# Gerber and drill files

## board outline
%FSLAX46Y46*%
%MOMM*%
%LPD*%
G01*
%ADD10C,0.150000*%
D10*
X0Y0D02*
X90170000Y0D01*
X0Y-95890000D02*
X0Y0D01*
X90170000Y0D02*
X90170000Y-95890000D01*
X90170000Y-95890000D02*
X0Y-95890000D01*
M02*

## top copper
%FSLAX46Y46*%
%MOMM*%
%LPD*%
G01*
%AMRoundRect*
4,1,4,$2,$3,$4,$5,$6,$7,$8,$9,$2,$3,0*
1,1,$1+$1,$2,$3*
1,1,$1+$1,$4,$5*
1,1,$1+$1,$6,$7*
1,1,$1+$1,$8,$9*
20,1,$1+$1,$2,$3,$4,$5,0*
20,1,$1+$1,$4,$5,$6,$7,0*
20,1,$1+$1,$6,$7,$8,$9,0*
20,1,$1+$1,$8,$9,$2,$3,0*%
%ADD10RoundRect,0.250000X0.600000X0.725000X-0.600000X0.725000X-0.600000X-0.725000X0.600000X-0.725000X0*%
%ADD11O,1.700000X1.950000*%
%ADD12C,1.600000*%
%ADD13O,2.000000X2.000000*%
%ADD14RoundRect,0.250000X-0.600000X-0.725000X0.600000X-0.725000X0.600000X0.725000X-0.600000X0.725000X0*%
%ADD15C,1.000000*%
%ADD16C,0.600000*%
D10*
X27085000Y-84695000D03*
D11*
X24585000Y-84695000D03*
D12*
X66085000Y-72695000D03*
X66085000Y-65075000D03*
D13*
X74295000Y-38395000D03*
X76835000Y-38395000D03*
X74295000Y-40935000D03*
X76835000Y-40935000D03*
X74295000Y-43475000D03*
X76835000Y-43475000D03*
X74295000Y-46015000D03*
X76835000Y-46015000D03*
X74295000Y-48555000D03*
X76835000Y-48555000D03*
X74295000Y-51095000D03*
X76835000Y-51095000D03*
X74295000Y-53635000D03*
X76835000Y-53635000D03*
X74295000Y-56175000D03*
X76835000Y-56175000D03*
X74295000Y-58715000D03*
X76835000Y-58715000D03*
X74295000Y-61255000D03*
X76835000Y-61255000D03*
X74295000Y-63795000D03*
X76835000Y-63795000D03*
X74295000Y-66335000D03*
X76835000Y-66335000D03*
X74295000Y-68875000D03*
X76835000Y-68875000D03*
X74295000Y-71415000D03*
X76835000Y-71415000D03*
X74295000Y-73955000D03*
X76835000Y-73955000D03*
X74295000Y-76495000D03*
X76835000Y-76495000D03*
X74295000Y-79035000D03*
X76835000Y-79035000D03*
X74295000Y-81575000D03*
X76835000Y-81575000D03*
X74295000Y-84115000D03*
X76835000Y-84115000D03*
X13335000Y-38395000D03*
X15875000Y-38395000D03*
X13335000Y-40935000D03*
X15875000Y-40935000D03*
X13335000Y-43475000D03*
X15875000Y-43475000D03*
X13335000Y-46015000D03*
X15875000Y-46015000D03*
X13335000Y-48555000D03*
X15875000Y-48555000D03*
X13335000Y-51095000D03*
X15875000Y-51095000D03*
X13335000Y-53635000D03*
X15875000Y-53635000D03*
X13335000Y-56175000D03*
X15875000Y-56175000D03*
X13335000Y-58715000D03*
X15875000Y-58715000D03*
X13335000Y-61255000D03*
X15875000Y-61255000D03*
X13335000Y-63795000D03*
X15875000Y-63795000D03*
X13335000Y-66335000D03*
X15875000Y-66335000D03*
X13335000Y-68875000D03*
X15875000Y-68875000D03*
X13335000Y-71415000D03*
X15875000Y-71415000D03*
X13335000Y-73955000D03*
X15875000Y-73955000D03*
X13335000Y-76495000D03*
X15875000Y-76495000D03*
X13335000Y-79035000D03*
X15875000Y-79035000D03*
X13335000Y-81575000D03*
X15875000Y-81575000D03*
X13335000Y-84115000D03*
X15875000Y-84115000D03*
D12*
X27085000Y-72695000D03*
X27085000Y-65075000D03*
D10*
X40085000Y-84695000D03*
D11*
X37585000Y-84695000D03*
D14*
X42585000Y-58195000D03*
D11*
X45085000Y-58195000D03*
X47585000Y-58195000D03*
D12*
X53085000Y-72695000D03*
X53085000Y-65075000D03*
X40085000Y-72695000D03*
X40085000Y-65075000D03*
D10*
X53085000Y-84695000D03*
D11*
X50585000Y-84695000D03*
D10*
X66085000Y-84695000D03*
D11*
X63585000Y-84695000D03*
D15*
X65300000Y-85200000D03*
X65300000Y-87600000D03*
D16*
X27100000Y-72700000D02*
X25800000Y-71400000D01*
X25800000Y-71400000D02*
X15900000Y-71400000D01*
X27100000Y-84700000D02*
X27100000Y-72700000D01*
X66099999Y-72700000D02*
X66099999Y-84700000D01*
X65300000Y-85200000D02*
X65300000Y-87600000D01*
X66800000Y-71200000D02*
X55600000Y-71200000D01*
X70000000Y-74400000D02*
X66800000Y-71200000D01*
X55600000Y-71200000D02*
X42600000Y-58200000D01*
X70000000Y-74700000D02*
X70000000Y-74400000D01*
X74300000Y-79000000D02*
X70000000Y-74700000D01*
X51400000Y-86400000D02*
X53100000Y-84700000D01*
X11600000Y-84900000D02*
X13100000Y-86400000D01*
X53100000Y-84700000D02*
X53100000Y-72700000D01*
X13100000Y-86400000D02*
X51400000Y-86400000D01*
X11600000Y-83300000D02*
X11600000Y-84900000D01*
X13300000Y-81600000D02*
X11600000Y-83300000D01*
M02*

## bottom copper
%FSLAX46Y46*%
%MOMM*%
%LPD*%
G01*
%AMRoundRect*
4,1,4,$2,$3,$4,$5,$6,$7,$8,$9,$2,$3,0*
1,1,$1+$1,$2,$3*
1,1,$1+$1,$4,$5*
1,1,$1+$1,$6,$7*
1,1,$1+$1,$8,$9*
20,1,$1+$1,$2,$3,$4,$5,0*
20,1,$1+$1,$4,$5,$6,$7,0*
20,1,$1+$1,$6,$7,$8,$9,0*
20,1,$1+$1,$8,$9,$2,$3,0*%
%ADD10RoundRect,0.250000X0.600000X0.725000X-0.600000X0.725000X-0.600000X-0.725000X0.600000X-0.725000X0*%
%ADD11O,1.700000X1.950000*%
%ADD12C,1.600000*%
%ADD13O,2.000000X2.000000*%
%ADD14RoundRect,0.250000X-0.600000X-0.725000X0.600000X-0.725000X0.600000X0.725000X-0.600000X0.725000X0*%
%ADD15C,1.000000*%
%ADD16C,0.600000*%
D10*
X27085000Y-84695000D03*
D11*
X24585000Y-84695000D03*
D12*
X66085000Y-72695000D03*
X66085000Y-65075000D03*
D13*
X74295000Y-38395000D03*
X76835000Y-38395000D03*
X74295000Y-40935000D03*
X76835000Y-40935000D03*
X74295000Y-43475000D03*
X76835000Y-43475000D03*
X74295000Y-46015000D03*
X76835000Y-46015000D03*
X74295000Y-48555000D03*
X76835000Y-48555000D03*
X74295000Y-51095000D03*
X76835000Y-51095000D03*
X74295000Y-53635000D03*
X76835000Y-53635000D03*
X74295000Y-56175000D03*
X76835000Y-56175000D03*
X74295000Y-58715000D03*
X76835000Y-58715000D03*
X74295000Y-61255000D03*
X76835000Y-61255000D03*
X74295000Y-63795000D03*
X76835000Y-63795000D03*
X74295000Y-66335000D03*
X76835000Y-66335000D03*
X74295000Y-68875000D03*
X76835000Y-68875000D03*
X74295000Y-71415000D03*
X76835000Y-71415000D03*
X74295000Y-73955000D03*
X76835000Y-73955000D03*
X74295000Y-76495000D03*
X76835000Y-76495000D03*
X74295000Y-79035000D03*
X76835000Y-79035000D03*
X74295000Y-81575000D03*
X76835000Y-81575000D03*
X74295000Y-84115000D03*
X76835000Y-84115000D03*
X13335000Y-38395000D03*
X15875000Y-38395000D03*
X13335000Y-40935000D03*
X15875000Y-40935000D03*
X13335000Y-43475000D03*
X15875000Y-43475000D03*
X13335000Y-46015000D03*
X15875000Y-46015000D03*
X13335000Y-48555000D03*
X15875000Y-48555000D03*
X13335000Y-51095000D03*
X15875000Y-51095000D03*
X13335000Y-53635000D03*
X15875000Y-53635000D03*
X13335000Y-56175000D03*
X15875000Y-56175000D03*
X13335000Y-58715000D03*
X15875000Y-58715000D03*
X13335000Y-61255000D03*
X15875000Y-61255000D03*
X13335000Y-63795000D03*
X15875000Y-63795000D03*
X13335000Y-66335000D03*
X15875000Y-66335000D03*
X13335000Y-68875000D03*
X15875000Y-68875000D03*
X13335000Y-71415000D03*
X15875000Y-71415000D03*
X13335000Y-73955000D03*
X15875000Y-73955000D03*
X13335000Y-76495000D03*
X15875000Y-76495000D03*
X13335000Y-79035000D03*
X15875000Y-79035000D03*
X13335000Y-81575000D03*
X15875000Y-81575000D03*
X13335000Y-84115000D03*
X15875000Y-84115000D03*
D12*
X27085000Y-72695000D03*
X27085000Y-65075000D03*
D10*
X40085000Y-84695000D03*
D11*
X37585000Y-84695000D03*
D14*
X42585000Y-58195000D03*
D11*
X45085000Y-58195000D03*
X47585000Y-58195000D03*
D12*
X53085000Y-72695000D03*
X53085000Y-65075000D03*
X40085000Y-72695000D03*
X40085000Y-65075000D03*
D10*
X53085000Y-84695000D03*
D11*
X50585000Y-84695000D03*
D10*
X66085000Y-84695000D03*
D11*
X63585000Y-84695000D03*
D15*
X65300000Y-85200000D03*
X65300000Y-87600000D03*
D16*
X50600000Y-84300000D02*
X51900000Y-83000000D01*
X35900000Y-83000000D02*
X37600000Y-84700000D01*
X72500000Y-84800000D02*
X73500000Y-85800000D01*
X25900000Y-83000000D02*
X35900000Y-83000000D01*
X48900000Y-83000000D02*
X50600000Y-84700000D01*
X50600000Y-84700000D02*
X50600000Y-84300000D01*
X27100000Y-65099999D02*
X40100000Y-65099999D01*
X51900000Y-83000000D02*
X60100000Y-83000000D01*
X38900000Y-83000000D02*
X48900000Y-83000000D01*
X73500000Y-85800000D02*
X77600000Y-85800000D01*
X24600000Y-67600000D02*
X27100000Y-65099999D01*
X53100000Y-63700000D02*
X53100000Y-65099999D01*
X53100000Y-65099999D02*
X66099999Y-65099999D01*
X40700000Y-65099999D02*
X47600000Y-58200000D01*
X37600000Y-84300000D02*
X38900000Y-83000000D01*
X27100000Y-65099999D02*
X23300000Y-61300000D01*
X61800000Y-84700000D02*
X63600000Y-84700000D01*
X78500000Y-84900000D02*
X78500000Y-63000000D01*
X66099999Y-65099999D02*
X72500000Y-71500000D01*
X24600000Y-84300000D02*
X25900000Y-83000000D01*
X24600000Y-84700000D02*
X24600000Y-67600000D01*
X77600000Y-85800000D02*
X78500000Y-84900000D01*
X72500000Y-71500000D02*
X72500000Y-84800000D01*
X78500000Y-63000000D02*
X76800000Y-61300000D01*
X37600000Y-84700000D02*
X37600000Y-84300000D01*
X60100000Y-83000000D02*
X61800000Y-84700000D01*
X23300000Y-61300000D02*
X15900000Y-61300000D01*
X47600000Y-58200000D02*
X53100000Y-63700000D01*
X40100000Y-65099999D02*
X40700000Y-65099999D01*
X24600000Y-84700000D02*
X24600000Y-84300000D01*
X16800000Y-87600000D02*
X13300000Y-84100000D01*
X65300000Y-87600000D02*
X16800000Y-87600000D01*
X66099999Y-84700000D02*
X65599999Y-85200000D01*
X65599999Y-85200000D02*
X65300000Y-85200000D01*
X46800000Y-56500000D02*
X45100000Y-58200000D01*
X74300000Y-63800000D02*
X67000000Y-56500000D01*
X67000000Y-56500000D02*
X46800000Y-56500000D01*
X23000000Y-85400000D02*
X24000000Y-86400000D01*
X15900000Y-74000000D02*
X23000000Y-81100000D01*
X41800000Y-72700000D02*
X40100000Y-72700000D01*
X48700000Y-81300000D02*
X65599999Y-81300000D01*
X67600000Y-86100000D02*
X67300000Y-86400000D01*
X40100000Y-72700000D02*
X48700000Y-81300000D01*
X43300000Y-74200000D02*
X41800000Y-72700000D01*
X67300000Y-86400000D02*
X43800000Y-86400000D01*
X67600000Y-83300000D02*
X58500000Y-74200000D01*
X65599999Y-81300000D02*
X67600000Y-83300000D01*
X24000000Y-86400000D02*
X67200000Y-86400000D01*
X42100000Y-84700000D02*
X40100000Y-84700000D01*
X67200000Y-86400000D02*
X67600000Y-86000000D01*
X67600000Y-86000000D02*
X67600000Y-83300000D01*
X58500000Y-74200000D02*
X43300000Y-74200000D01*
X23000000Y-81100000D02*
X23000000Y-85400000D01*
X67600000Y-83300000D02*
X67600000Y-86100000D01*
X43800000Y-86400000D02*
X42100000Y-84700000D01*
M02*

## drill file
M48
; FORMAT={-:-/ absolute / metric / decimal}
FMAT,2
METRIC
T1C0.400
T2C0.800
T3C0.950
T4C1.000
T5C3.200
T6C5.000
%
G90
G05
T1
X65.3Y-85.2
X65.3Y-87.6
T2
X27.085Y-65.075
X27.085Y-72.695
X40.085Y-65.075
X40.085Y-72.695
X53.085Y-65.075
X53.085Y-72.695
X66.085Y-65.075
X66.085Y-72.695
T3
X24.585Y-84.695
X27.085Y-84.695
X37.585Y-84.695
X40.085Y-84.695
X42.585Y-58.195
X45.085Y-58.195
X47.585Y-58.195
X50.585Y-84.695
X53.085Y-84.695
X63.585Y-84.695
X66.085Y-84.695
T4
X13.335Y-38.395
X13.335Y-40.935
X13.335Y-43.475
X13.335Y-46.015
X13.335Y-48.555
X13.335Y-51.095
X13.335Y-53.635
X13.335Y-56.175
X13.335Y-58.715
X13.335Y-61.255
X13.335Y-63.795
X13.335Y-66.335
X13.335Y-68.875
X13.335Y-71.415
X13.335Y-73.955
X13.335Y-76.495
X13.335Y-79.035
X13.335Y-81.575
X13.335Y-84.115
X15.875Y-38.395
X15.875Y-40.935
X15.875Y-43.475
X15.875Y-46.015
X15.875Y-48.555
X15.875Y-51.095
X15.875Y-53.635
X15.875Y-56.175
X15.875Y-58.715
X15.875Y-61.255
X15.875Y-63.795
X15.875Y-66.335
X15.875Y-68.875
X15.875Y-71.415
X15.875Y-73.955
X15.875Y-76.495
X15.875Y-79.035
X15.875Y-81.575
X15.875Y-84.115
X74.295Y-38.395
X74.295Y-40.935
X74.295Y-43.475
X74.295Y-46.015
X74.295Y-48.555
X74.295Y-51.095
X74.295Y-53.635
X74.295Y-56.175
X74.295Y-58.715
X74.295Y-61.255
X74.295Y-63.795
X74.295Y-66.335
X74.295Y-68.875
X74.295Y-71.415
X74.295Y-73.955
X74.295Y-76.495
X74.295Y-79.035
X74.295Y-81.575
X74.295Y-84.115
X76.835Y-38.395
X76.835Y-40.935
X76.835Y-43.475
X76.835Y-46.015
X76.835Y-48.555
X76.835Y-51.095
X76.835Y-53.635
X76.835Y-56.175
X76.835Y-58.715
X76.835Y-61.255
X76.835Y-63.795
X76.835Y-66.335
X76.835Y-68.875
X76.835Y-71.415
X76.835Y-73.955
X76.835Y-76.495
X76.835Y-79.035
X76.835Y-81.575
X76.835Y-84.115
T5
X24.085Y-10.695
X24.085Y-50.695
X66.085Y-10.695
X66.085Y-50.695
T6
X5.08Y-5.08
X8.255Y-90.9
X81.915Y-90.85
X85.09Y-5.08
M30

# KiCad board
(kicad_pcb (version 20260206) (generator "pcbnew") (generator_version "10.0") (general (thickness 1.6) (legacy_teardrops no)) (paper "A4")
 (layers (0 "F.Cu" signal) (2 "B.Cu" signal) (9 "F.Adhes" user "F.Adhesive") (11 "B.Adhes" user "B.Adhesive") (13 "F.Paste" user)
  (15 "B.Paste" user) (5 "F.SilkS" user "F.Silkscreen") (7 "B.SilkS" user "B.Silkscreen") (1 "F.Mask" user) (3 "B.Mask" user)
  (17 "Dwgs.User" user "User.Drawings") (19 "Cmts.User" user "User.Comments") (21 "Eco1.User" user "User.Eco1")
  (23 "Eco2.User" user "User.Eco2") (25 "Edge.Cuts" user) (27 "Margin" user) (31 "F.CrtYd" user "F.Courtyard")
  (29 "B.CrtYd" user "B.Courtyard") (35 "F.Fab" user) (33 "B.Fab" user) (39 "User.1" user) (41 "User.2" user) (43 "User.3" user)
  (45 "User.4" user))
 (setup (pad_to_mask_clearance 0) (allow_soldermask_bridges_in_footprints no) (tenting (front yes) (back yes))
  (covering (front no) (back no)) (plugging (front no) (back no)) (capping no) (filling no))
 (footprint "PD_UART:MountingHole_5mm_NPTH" (layer "F.Cu") (at 8.255 90.9)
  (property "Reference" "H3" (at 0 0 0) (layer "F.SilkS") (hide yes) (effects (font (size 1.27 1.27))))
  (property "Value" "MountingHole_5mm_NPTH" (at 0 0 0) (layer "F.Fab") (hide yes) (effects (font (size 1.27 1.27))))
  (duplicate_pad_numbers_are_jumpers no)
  (pad "" np_thru_hole circle (at 0 0) (size 5 5) (drill 5) (layers "*.Cu")))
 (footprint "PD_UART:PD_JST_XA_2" (layer "F.Cu") (at 27.085 84.695 180)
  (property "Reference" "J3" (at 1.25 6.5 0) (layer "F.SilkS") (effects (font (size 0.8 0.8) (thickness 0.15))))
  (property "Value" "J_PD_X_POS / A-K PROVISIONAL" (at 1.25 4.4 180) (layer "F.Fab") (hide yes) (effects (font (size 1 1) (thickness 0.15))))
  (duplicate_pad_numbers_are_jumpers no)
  (pad "1" thru_hole roundrect (at 0 0 180) (size 1.7 1.95) (drill 0.95) (layers "*.Cu") (remove_unused_layers no)
   (roundrect_rratio 0.147059) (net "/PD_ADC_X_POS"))
  (pad "2" thru_hole oval (at 2.5 0 180) (size 1.7 1.95) (drill 0.95) (layers "*.Cu") (remove_unused_layers no) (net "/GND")))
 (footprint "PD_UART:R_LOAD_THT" (layer "F.Cu") (at 66.085 72.695 90)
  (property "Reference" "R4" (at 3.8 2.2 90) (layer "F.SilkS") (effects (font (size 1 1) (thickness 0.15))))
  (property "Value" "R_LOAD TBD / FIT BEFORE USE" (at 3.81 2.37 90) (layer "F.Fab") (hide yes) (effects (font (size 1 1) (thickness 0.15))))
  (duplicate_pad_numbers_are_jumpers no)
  (pad "1" thru_hole circle (at 0 0 90) (size 1.6 1.6) (drill 0.8) (layers "*.Cu") (remove_unused_layers no) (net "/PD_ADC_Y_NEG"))
  (pad "2" thru_hole circle (at 7.62 0 90) (size 1.6 1.6) (drill 0.8) (layers "*.Cu") (remove_unused_layers no) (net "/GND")))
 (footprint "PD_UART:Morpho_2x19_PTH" (layer "F.Cu") (at 74.295 38.395)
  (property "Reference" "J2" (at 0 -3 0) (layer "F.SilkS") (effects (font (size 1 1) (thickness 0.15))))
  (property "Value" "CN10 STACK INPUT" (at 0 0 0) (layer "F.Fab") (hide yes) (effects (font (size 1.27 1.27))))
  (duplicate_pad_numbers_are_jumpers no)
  (pad "1" thru_hole oval (at 0 0) (size 2 2) (drill 1) (layers "*.Cu") (remove_unused_layers no) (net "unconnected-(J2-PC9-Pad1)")
   (thermal_bridge_angle 45))
  (pad "2" thru_hole oval (at 2.54 0) (size 2 2) (drill 1) (layers "*.Cu") (remove_unused_layers no) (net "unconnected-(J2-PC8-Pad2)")
   (thermal_bridge_angle 45))
  (pad "3" thru_hole oval (at 0 2.54) (size 2 2) (drill 1) (layers "*.Cu") (remove_unused_layers no) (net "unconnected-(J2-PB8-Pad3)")
   (thermal_bridge_angle 45))
  (pad "4" thru_hole oval (at 2.54 2.54) (size 2 2) (drill 1) (layers "*.Cu") (remove_unused_layers no) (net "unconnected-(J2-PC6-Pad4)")
   (thermal_bridge_angle 45))
  (pad "5" thru_hole oval (at 0 5.08) (size 2 2) (drill 1) (layers "*.Cu") (remove_unused_layers no) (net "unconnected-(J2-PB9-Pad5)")
   (thermal_bridge_angle 45))
  (pad "6" thru_hole oval (at 2.54 5.08) (size 2 2) (drill 1) (layers "*.Cu") (remove_unused_layers no) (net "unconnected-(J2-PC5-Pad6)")
   (thermal_bridge_angle 45))
  (pad "7" thru_hole oval (at 0 7.62) (size 2 2) (drill 1) (layers "*.Cu") (remove_unused_layers no) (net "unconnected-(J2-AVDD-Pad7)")
   (thermal_bridge_angle 45))
  (pad "8" thru_hole oval (at 2.54 7.62) (size 2 2) (drill 1) (layers "*.Cu") (remove_unused_layers no) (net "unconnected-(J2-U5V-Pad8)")
   (thermal_bridge_angle 45))
  (pad "9" thru_hole oval (at 0 10.16) (size 2 2) (drill 1) (layers "*.Cu") (remove_unused_layers no) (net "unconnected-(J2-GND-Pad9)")
   (thermal_bridge_angle 45))
  (pad "10" thru_hole oval (at 2.54 10.16) (size 2 2) (drill 1) (layers "*.Cu") (remove_unused_layers no) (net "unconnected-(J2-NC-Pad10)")
   (thermal_bridge_angle 45))
  (pad "11" thru_hole oval (at 0 12.7) (size 2 2) (drill 1) (layers "*.Cu") (remove_unused_layers no) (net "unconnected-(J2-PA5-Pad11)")
   (thermal_bridge_angle 45))
  (pad "12" thru_hole oval (at 2.54 12.7) (size 2 2) (drill 1) (layers "*.Cu") (remove_unused_layers no) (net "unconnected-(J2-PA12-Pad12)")
   (thermal_bridge_angle 45))
  (pad "13" thru_hole oval (at 0 15.24) (size 2 2) (drill 1) (layers "*.Cu") (remove_unused_layers no) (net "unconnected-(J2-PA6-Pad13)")
   (thermal_bridge_angle 45))
  (pad "14" thru_hole oval (at 2.54 15.24) (size 2 2) (drill 1) (layers "*.Cu") (remove_unused_layers no)
   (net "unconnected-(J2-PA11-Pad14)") (thermal_bridge_angle 45))
  (pad "15" thru_hole oval (at 0 17.78) (size 2 2) (drill 1) (layers "*.Cu") (remove_unused_layers no) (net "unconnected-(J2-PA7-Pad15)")
   (thermal_bridge_angle 45))
  (pad "16" thru_hole oval (at 2.54 17.78) (size 2 2) (drill 1) (layers "*.Cu") (remove_unused_layers no)
   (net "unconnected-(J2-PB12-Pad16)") (thermal_bridge_angle 45))
  (pad "17" thru_hole oval (at 0 20.32) (size 2 2) (drill 1) (layers "*.Cu") (remove_unused_layers no) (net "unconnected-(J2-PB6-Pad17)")
   (thermal_bridge_angle 45))
  (pad "18" thru_hole oval (at 2.54 20.32) (size 2 2) (drill 1) (layers "*.Cu") (remove_unused_layers no)
   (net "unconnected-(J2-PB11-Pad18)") (thermal_bridge_angle 45))
  (pad "19" thru_hole oval (at 0 22.86) (size 2 2) (drill 1) (layers "*.Cu") (remove_unused_layers no) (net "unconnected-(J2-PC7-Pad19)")
   (thermal_bridge_angle 45))
  (pad "20" thru_hole oval (at 2.54 22.86) (size 2 2) (drill 1) (layers "*.Cu") (remove_unused_layers no) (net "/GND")
   (thermal_bridge_angle 45))
  (pad "21" thru_hole oval (at 0 25.4) (size 2 2) (drill 1) (layers "*.Cu") (remove_unused_layers no) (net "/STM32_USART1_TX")
   (thermal_bridge_angle 45))
  (pad "22" thru_hole oval (at 2.54 25.4) (size 2 2) (drill 1) (layers "*.Cu") (remove_unused_layers no) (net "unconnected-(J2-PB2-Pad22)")
   (thermal_bridge_angle 45))
  (pad "23" thru_hole oval (at 0 27.94) (size 2 2) (drill 1) (layers "*.Cu") (remove_unused_layers no) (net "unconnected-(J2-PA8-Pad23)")
   (thermal_bridge_angle 45))
  (pad "24" thru_hole oval (at 2.54 27.94) (size 2 2) (drill 1) (layers "*.Cu") (remove_unused_layers no) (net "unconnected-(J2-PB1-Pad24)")
   (thermal_bridge_angle 45))
  (pad "25" thru_hole oval (at 0 30.48) (size 2 2) (drill 1) (layers "*.Cu") (remove_unused_layers no) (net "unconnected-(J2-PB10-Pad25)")
   (thermal_bridge_angle 45))
  (pad "26" thru_hole oval (at 2.54 30.48) (size 2 2) (drill 1) (layers "*.Cu") (remove_unused_layers no)
   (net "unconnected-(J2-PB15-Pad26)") (thermal_bridge_angle 45))
  (pad "27" thru_hole oval (at 0 33.02) (size 2 2) (drill 1) (layers "*.Cu") (remove_unused_layers no) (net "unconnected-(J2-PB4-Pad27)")
   (thermal_bridge_angle 45))
  (pad "28" thru_hole oval (at 2.54 33.02) (size 2 2) (drill 1) (layers "*.Cu") (remove_unused_layers no)
   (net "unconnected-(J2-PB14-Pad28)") (thermal_bridge_angle 45))
  (pad "29" thru_hole oval (at 0 35.56) (size 2 2) (drill 1) (layers "*.Cu") (remove_unused_layers no) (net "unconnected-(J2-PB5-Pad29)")
   (thermal_bridge_angle 45))
  (pad "30" thru_hole oval (at 2.54 35.56) (size 2 2) (drill 1) (layers "*.Cu") (remove_unused_layers no)
   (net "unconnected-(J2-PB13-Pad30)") (thermal_bridge_angle 45))
  (pad "31" thru_hole oval (at 0 38.1) (size 2 2) (drill 1) (layers "*.Cu") (remove_unused_layers no) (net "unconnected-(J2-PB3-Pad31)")
   (thermal_bridge_angle 45))
  (pad "32" thru_hole oval (at 2.54 38.1) (size 2 2) (drill 1) (layers "*.Cu") (remove_unused_layers no) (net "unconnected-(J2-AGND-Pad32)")
   (thermal_bridge_angle 45))
  (pad "33" thru_hole oval (at 0 40.64) (size 2 2) (drill 1) (layers "*.Cu") (remove_unused_layers no) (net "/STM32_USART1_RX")
   (thermal_bridge_angle 45))
  (pad "34" thru_hole oval (at 2.54 40.64) (size 2 2) (drill 1) (layers "*.Cu") (remove_unused_layers no) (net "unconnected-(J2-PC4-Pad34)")
   (thermal_bridge_angle 45))
  (pad "35" thru_hole oval (at 0 43.18) (size 2 2) (drill 1) (layers "*.Cu") (remove_unused_layers no) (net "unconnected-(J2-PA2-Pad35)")
   (thermal_bridge_angle 45))
  (pad "36" thru_hole oval (at 2.54 43.18) (size 2 2) (drill 1) (layers "*.Cu") (remove_unused_layers no) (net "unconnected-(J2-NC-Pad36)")
   (thermal_bridge_angle 45))
  (pad "37" thru_hole oval (at 0 45.72) (size 2 2) (drill 1) (layers "*.Cu") (remove_unused_layers no) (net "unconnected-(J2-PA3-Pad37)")
   (thermal_bridge_angle 45))
  (pad "38" thru_hole oval (at 2.54 45.72) (size 2 2) (drill 1) (layers "*.Cu") (remove_unused_layers no) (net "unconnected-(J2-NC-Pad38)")
   (thermal_bridge_angle 45)))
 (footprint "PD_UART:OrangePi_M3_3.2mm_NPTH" (layer "F.Cu") (at 66.085 10.695)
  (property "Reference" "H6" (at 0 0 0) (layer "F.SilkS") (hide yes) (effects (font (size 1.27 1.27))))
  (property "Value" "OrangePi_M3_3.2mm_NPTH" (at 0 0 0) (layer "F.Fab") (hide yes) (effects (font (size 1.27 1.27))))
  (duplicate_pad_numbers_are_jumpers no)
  (pad "" np_thru_hole circle (at 0 0) (size 3.2 3.2) (drill 3.2) (layers "*.Cu")))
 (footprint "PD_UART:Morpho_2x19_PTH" (layer "F.Cu") (at 13.335 38.395)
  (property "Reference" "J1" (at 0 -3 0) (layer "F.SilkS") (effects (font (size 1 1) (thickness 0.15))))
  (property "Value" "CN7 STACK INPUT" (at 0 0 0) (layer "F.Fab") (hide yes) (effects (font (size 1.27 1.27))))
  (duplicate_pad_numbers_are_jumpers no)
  (pad "1" thru_hole oval (at 0 0) (size 2 2) (drill 1) (layers "*.Cu") (remove_unused_layers no) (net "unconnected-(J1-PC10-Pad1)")
   (thermal_bridge_angle 45))
  (pad "2" thru_hole oval (at 2.54 0) (size 2 2) (drill 1) (layers "*.Cu") (remove_unused_layers no) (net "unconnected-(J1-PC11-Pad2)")
   (thermal_bridge_angle 45))
  (pad "3" thru_hole oval (at 0 2.54) (size 2 2) (drill 1) (layers "*.Cu") (remove_unused_layers no) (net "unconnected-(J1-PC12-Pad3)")
   (thermal_bridge_angle 45))
  (pad "4" thru_hole oval (at 2.54 2.54) (size 2 2) (drill 1) (layers "*.Cu") (remove_unused_layers no) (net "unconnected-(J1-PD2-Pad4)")
   (thermal_bridge_angle 45))
  (pad "5" thru_hole oval (at 0 5.08) (size 2 2) (drill 1) (layers "*.Cu") (remove_unused_layers no) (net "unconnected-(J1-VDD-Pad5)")
   (thermal_bridge_angle 45))
  (pad "6" thru_hole oval (at 2.54 5.08) (size 2 2) (drill 1) (layers "*.Cu") (remove_unused_layers no) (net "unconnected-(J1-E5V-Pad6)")
   (thermal_bridge_angle 45))
  (pad "7" thru_hole oval (at 0 7.62) (size 2 2) (drill 1) (layers "*.Cu") (remove_unused_layers no) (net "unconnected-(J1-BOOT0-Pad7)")
   (thermal_bridge_angle 45))
  (pad "8" thru_hole oval (at 2.54 7.62) (size 2 2) (drill 1) (layers "*.Cu") (remove_unused_layers no) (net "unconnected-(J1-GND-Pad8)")
   (thermal_bridge_angle 45))
  (pad "9" thru_hole oval (at 0 10.16) (size 2 2) (drill 1) (layers "*.Cu") (remove_unused_layers no) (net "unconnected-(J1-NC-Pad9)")
   (thermal_bridge_angle 45))
  (pad "10" thru_hole oval (at 2.54 10.16) (size 2 2) (drill 1) (layers "*.Cu") (remove_unused_layers no) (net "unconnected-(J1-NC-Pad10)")
   (thermal_bridge_angle 45))
  (pad "11" thru_hole oval (at 0 12.7) (size 2 2) (drill 1) (layers "*.Cu") (remove_unused_layers no) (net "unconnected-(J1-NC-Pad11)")
   (thermal_bridge_angle 45))
  (pad "12" thru_hole oval (at 2.54 12.7) (size 2 2) (drill 1) (layers "*.Cu") (remove_unused_layers no)
   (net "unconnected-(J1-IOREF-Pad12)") (thermal_bridge_angle 45))
  (pad "13" thru_hole oval (at 0 15.24) (size 2 2) (drill 1) (layers "*.Cu") (remove_unused_layers no) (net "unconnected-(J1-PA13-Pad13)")
   (thermal_bridge_angle 45))
  (pad "14" thru_hole oval (at 2.54 15.24) (size 2 2) (drill 1) (layers "*.Cu") (remove_unused_layers no)
   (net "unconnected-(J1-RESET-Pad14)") (thermal_bridge_angle 45))
  (pad "15" thru_hole oval (at 0 17.78) (size 2 2) (drill 1) (layers "*.Cu") (remove_unused_layers no) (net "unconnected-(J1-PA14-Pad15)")
   (thermal_bridge_angle 45))
  (pad "16" thru_hole oval (at 2.54 17.78) (size 2 2) (drill 1) (layers "*.Cu") (remove_unused_layers no) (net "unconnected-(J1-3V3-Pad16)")
   (thermal_bridge_angle 45))
  (pad "17" thru_hole oval (at 0 20.32) (size 2 2) (drill 1) (layers "*.Cu") (remove_unused_layers no) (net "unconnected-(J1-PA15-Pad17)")
   (thermal_bridge_angle 45))
  (pad "18" thru_hole oval (at 2.54 20.32) (size 2 2) (drill 1) (layers "*.Cu") (remove_unused_layers no) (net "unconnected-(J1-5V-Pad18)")
   (thermal_bridge_angle 45))
  (pad "19" thru_hole oval (at 0 22.86) (size 2 2) (drill 1) (layers "*.Cu") (remove_unused_layers no) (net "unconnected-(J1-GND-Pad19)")
   (thermal_bridge_angle 45))
  (pad "20" thru_hole oval (at 2.54 22.86) (size 2 2) (drill 1) (layers "*.Cu") (remove_unused_layers no) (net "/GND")
   (thermal_bridge_angle 45))
  (pad "21" thru_hole oval (at 0 25.4) (size 2 2) (drill 1) (layers "*.Cu") (remove_unused_layers no) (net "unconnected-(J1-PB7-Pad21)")
   (thermal_bridge_angle 45))
  (pad "22" thru_hole oval (at 2.54 25.4) (size 2 2) (drill 1) (layers "*.Cu") (remove_unused_layers no) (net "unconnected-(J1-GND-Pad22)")
   (thermal_bridge_angle 45))
  (pad "23" thru_hole oval (at 0 27.94) (size 2 2) (drill 1) (layers "*.Cu") (remove_unused_layers no) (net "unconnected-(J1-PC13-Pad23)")
   (thermal_bridge_angle 45))
  (pad "24" thru_hole oval (at 2.54 27.94) (size 2 2) (drill 1) (layers "*.Cu") (remove_unused_layers no) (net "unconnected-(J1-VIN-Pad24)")
   (thermal_bridge_angle 45))
  (pad "25" thru_hole oval (at 0 30.48) (size 2 2) (drill 1) (layers "*.Cu") (remove_unused_layers no) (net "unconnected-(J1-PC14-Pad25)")
   (thermal_bridge_angle 45))
  (pad "26" thru_hole oval (at 2.54 30.48) (size 2 2) (drill 1) (layers "*.Cu") (remove_unused_layers no) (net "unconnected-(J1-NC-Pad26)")
   (thermal_bridge_angle 45))
  (pad "27" thru_hole oval (at 0 33.02) (size 2 2) (drill 1) (layers "*.Cu") (remove_unused_layers no) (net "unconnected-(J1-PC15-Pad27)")
   (thermal_bridge_angle 45))
  (pad "28" thru_hole oval (at 2.54 33.02) (size 2 2) (drill 1) (layers "*.Cu") (remove_unused_layers no) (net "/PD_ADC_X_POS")
   (thermal_bridge_angle 45))
  (pad "29" thru_hole oval (at 0 35.56) (size 2 2) (drill 1) (layers "*.Cu") (remove_unused_layers no) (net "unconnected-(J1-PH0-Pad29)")
   (thermal_bridge_angle 45))
  (pad "30" thru_hole oval (at 2.54 35.56) (size 2 2) (drill 1) (layers "*.Cu") (remove_unused_layers no) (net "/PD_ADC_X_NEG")
   (thermal_bridge_angle 45))
  (pad "31" thru_hole oval (at 0 38.1) (size 2 2) (drill 1) (layers "*.Cu") (remove_unused_layers no) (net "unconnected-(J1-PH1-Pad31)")
   (thermal_bridge_angle 45))
  (pad "32" thru_hole oval (at 2.54 38.1) (size 2 2) (drill 1) (layers "*.Cu") (remove_unused_layers no) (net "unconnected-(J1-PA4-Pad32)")
   (thermal_bridge_angle 45))
  (pad "33" thru_hole oval (at 0 40.64) (size 2 2) (drill 1) (layers "*.Cu") (remove_unused_layers no) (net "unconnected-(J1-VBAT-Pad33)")
   (thermal_bridge_angle 45))
  (pad "34" thru_hole oval (at 2.54 40.64) (size 2 2) (drill 1) (layers "*.Cu") (remove_unused_layers no) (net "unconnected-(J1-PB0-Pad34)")
   (thermal_bridge_angle 45))
  (pad "35" thru_hole oval (at 0 43.18) (size 2 2) (drill 1) (layers "*.Cu") (remove_unused_layers no) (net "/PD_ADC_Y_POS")
   (thermal_bridge_angle 45))
  (pad "36" thru_hole oval (at 2.54 43.18) (size 2 2) (drill 1) (layers "*.Cu") (remove_unused_layers no)
   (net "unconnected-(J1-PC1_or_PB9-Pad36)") (thermal_bridge_angle 45))
  (pad "37" thru_hole oval (at 0 45.72) (size 2 2) (drill 1) (layers "*.Cu") (remove_unused_layers no) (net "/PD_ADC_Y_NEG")
   (thermal_bridge_angle 45))
  (pad "38" thru_hole oval (at 2.54 45.72) (size 2 2) (drill 1) (layers "*.Cu") (remove_unused_layers no) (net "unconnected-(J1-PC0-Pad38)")
   (thermal_bridge_angle 45)))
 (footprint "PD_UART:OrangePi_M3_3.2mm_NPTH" (layer "F.Cu") (at 24.085 50.695)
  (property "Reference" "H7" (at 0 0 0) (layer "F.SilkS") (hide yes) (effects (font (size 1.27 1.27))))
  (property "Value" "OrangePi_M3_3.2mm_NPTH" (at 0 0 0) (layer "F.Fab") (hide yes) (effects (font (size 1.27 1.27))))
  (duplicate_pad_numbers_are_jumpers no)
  (pad "" np_thru_hole circle (at 0 0) (size 3.2 3.2) (drill 3.2) (layers "*.Cu")))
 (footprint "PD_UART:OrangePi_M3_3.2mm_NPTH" (layer "F.Cu") (at 24.085 10.695)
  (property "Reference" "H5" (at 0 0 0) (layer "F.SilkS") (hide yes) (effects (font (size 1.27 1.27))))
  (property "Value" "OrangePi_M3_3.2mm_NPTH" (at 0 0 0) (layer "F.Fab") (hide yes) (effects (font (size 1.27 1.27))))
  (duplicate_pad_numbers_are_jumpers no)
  (pad "" np_thru_hole circle (at 0 0) (size 3.2 3.2) (drill 3.2) (layers "*.Cu")))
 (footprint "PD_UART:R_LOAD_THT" (layer "F.Cu") (at 27.085 72.695 90)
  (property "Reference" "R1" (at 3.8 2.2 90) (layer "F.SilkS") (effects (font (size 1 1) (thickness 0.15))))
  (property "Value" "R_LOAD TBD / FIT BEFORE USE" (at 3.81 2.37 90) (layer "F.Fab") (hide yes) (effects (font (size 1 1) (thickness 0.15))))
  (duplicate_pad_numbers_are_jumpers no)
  (pad "1" thru_hole circle (at 0 0 90) (size 1.6 1.6) (drill 0.8) (layers "*.Cu") (remove_unused_layers no) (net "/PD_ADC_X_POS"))
  (pad "2" thru_hole circle (at 7.62 0 90) (size 1.6 1.6) (drill 0.8) (layers "*.Cu") (remove_unused_layers no) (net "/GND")))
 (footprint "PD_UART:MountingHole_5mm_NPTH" (layer "F.Cu") (at 81.915 90.85)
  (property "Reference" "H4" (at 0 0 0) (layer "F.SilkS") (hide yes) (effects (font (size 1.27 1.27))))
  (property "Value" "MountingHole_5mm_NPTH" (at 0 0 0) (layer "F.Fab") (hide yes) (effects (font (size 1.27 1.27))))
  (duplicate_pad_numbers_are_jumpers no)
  (pad "" np_thru_hole circle (at 0 0) (size 5 5) (drill 5) (layers "*.Cu")))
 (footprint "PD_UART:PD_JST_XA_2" (layer "F.Cu") (at 40.085 84.695 180)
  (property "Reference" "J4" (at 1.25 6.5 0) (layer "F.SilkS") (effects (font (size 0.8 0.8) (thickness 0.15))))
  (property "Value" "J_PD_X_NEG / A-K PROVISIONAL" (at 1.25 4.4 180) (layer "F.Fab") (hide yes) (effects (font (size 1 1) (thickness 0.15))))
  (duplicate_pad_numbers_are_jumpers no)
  (pad "1" thru_hole roundrect (at 0 0 180) (size 1.7 1.95) (drill 0.95) (layers "*.Cu") (remove_unused_layers no)
   (roundrect_rratio 0.147059) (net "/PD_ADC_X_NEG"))
  (pad "2" thru_hole oval (at 2.5 0 180) (size 1.7 1.95) (drill 0.95) (layers "*.Cu") (remove_unused_layers no) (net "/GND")))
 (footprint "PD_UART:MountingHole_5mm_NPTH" (layer "F.Cu") (at 85.09 5.08)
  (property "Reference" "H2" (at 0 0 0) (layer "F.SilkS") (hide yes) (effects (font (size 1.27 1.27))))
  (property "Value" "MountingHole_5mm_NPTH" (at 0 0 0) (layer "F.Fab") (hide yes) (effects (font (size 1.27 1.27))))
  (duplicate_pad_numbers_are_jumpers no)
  (pad "" np_thru_hole circle (at 0 0) (size 5 5) (drill 5) (layers "*.Cu")))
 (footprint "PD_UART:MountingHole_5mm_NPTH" (layer "F.Cu") (at 5.08 5.08)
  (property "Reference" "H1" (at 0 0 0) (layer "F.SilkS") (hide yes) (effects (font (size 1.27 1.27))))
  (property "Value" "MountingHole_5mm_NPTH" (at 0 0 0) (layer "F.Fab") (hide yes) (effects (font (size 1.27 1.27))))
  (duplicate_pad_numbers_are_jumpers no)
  (pad "" np_thru_hole circle (at 0 0) (size 5 5) (drill 5) (layers "*.Cu")))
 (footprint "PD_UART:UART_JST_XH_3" (layer "F.Cu") (at 42.585 58.195)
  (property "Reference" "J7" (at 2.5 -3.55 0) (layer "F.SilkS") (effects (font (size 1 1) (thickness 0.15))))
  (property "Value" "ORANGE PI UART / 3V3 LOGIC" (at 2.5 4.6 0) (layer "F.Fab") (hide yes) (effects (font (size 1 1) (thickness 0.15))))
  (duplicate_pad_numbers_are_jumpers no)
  (pad "1" thru_hole roundrect (at 0 0) (size 1.7 1.95) (drill 0.95) (layers "*.Cu") (remove_unused_layers no) (roundrect_rratio 0.147059)
   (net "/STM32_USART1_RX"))
  (pad "2" thru_hole oval (at 2.5 0) (size 1.7 1.95) (drill 0.95) (layers "*.Cu") (remove_unused_layers no) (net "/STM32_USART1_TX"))
  (pad "3" thru_hole oval (at 5 0) (size 1.7 1.95) (drill 0.95) (layers "*.Cu") (remove_unused_layers no) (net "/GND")))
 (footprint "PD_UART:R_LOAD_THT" (layer "F.Cu") (at 53.085 72.695 90)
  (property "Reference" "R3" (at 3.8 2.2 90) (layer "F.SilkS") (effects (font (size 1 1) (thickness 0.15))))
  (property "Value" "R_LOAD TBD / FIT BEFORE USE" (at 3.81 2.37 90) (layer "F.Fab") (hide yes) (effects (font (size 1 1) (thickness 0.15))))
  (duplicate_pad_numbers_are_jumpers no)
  (pad "1" thru_hole circle (at 0 0 90) (size 1.6 1.6) (drill 0.8) (layers "*.Cu") (remove_unused_layers no) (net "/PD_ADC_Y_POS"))
  (pad "2" thru_hole circle (at 7.62 0 90) (size 1.6 1.6) (drill 0.8) (layers "*.Cu") (remove_unused_layers no) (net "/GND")))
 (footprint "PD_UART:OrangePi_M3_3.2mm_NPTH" (layer "F.Cu") (at 66.085 50.695)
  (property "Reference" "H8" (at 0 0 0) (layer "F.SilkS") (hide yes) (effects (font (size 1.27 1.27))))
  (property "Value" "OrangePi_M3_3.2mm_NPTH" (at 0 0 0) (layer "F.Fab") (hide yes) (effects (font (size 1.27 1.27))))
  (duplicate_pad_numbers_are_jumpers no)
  (pad "" np_thru_hole circle (at 0 0) (size 3.2 3.2) (drill 3.2) (layers "*.Cu")))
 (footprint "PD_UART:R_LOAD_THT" (layer "F.Cu") (at 40.085 72.695 90)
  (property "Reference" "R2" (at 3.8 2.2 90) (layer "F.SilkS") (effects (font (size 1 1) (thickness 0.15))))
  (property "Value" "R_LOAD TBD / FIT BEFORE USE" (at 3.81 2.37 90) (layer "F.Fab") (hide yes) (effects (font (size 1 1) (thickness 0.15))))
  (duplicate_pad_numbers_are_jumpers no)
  (pad "1" thru_hole circle (at 0 0 90) (size 1.6 1.6) (drill 0.8) (layers "*.Cu") (remove_unused_layers no) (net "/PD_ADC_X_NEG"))
  (pad "2" thru_hole circle (at 7.62 0 90) (size 1.6 1.6) (drill 0.8) (layers "*.Cu") (remove_unused_layers no) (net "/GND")))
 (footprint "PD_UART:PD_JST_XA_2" (layer "F.Cu") (at 53.085 84.695 180)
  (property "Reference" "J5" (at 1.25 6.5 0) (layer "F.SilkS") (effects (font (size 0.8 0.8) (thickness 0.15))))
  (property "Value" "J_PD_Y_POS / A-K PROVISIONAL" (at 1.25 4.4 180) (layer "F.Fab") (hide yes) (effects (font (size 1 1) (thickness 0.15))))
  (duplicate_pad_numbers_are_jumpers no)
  (pad "1" thru_hole roundrect (at 0 0 180) (size 1.7 1.95) (drill 0.95) (layers "*.Cu") (remove_unused_layers no)
   (roundrect_rratio 0.147059) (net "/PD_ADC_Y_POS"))
  (pad "2" thru_hole oval (at 2.5 0 180) (size 1.7 1.95) (drill 0.95) (layers "*.Cu") (remove_unused_layers no) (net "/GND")))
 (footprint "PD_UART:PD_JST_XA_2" (layer "F.Cu") (at 66.085 84.695 180)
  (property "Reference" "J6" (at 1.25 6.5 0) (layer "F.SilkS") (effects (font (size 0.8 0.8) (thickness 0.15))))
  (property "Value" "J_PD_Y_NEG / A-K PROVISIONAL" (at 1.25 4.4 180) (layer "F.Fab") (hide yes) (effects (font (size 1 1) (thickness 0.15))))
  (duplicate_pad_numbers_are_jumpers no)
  (pad "1" thru_hole roundrect (at 0 0 180) (size 1.7 1.95) (drill 0.95) (layers "*.Cu") (remove_unused_layers no)
   (roundrect_rratio 0.147059) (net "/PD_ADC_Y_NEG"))
  (pad "2" thru_hole oval (at 2.5 0 180) (size 1.7 1.95) (drill 0.95) (layers "*.Cu") (remove_unused_layers no) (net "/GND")))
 (gr_line (start 0 0) (end 90.17 0) (stroke (width 0.15) (type default)) (layer "Edge.Cuts"))
 (gr_line (start 0 95.89) (end 0 0) (stroke (width 0.15) (type default)) (layer "Edge.Cuts"))
 (gr_line (start 90.17 0) (end 90.17 95.89) (stroke (width 0.15) (type default)) (layer "Edge.Cuts"))
 (gr_line (start 90.17 95.89) (end 0 95.89) (stroke (width 0.15) (type default)) (layer "Edge.Cuts"))
 (segment (start 27.1 72.7) (end 25.8 71.4) (width 0.6) (layer "F.Cu") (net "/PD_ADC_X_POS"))
 (segment (start 25.8 71.4) (end 15.9 71.4) (width 0.6) (layer "F.Cu") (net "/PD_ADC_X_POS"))
 (segment (start 27.1 84.7) (end 27.1 72.7) (width 0.6) (layer "F.Cu") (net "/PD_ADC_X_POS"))
 (segment (start 50.6 84.3) (end 51.9 83) (width 0.6) (layer "B.Cu") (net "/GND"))
 (segment (start 35.9 83) (end 37.6 84.7) (width 0.6) (layer "B.Cu") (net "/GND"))
 (segment (start 72.5 84.8) (end 73.5 85.8) (width 0.6) (layer "B.Cu") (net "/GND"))
 (segment (start 25.9 83) (end 35.9 83) (width 0.6) (layer "B.Cu") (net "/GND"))
 (segment (start 48.9 83) (end 50.6 84.7) (width 0.6) (layer "B.Cu") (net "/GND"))
 (segment (start 50.6 84.7) (end 50.6 84.3) (width 0.6) (layer "B.Cu") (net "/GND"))
 (segment (start 27.1 65.099999) (end 40.1 65.099999) (width 0.6) (layer "B.Cu") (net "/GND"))
 (segment (start 51.9 83) (end 60.1 83) (width 0.6) (layer "B.Cu") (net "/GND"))
 (segment (start 38.9 83) (end 48.9 83) (width 0.6) (layer "B.Cu") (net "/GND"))
 (segment (start 73.5 85.8) (end 77.6 85.8) (width 0.6) (layer "B.Cu") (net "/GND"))
 (segment (start 24.6 67.6) (end 27.1 65.099999) (width 0.6) (layer "B.Cu") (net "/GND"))
 (segment (start 53.1 63.7) (end 53.1 65.099999) (width 0.6) (layer "B.Cu") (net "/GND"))
 (segment (start 53.1 65.099999) (end 66.099999 65.099999) (width 0.6) (layer "B.Cu") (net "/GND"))
 (segment (start 40.7 65.099999) (end 47.6 58.2) (width 0.6) (layer "B.Cu") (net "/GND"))
 (segment (start 37.6 84.3) (end 38.9 83) (width 0.6) (layer "B.Cu") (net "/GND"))
 (segment (start 27.1 65.099999) (end 23.3 61.3) (width 0.6) (layer "B.Cu") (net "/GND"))
 (segment (start 61.8 84.7) (end 63.6 84.7) (width 0.6) (layer "B.Cu") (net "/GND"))
 (segment (start 78.5 84.9) (end 78.5 63) (width 0.6) (layer "B.Cu") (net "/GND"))
 (segment (start 66.099999 65.099999) (end 72.5 71.5) (width 0.6) (layer "B.Cu") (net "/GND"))
 (segment (start 24.6 84.3) (end 25.9 83) (width 0.6) (layer "B.Cu") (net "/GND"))
 (segment (start 24.6 84.7) (end 24.6 67.6) (width 0.6) (layer "B.Cu") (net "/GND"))
 (segment (start 77.6 85.8) (end 78.5 84.9) (width 0.6) (layer "B.Cu") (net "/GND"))
 (segment (start 72.5 71.5) (end 72.5 84.8) (width 0.6) (layer "B.Cu") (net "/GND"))
 (segment (start 78.5 63) (end 76.8 61.3) (width 0.6) (layer "B.Cu") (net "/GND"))
 (segment (start 37.6 84.7) (end 37.6 84.3) (width 0.6) (layer "B.Cu") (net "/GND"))
 (segment (start 60.1 83) (end 61.8 84.7) (width 0.6) (layer "B.Cu") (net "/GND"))
 (segment (start 23.3 61.3) (end 15.9 61.3) (width 0.6) (layer "B.Cu") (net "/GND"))
 (segment (start 47.6 58.2) (end 53.1 63.7) (width 0.6) (layer "B.Cu") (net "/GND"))
 (segment (start 40.1 65.099999) (end 40.7 65.099999) (width 0.6) (layer "B.Cu") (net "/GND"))
 (segment (start 24.6 84.7) (end 24.6 84.3) (width 0.6) (layer "B.Cu") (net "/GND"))
 (segment (start 66.099999 72.7) (end 66.099999 84.7) (width 0.6) (layer "F.Cu") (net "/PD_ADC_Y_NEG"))
 (segment (start 65.3 85.2) (end 65.3 87.6) (width 0.6) (layer "F.Cu") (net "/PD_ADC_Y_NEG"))
 (via (at 65.3 85.2) (size 1) (drill 0.4) (layers "F.Cu" "B.Cu") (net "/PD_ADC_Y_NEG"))
 (via (at 65.3 87.6) (size 1) (drill 0.4) (layers "F.Cu" "B.Cu") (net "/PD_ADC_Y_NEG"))
 (segment (start 16.8 87.6) (end 13.3 84.1) (width 0.6) (layer "B.Cu") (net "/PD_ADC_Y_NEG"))
 (segment (start 65.3 87.6) (end 16.8 87.6) (width 0.6) (layer "B.Cu") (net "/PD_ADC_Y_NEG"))
 (segment (start 66.099999 84.7) (end 65.599999 85.2) (width 0.6) (layer "B.Cu") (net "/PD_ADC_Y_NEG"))
 (segment (start 65.599999 85.2) (end 65.3 85.2) (width 0.6) (layer "B.Cu") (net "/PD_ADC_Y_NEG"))
 (segment (start 46.8 56.5) (end 45.1 58.2) (width 0.6) (layer "B.Cu") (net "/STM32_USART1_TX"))
 (segment (start 74.3 63.8) (end 67 56.5) (width 0.6) (layer "B.Cu") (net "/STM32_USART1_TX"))
 (segment (start 67 56.5) (end 46.8 56.5) (width 0.6) (layer "B.Cu") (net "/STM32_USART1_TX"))
 (segment (start 66.8 71.2) (end 55.6 71.2) (width 0.6) (layer "F.Cu") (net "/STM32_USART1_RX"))
 (segment (start 70 74.4) (end 66.8 71.2) (width 0.6) (layer "F.Cu") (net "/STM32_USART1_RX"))
 (segment (start 55.6 71.2) (end 42.6 58.2) (width 0.6) (layer "F.Cu") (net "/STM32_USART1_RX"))
 (segment (start 70 74.7) (end 70 74.4) (width 0.6) (layer "F.Cu") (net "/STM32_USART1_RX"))
 (segment (start 74.3 79) (end 70 74.7) (width 0.6) (layer "F.Cu") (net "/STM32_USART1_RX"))
 (segment (start 23 85.4) (end 24 86.4) (width 0.6) (layer "B.Cu") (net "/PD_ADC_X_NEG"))
 (segment (start 15.9 74) (end 23 81.1) (width 0.6) (layer "B.Cu") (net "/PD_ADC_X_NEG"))
 (segment (start 41.8 72.7) (end 40.1 72.7) (width 0.6) (layer "B.Cu") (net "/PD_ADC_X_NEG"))
 (segment (start 48.7 81.3) (end 65.599999 81.3) (width 0.6) (layer "B.Cu") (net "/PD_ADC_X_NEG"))
 (segment (start 67.6 86.1) (end 67.3 86.4) (width 0.6) (layer "B.Cu") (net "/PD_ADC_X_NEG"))
 (segment (start 40.1 72.7) (end 48.7 81.3) (width 0.6) (layer "B.Cu") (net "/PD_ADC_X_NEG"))
 (segment (start 43.3 74.2) (end 41.8 72.7) (width 0.6) (layer "B.Cu") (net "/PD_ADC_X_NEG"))
 (segment (start 67.3 86.4) (end 43.8 86.4) (width 0.6) (layer "B.Cu") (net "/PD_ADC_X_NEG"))
 (segment (start 67.6 83.3) (end 58.5 74.2) (width 0.6) (layer "B.Cu") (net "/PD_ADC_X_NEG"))
 (segment (start 65.599999 81.3) (end 67.6 83.3) (width 0.6) (layer "B.Cu") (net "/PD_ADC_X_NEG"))
 (segment (start 24 86.4) (end 67.2 86.4) (width 0.6) (layer "B.Cu") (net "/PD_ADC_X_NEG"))
 (segment (start 42.1 84.7) (end 40.1 84.7) (width 0.6) (layer "B.Cu") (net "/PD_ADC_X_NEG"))
 (segment (start 67.2 86.4) (end 67.6 86) (width 0.6) (layer "B.Cu") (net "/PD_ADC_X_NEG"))
 (segment (start 67.6 86) (end 67.6 83.3) (width 0.6) (layer "B.Cu") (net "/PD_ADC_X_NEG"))
 (segment (start 58.5 74.2) (end 43.3 74.2) (width 0.6) (layer "B.Cu") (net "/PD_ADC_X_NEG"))
 (segment (start 23 81.1) (end 23 85.4) (width 0.6) (layer "B.Cu") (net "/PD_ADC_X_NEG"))
 (segment (start 67.6 83.3) (end 67.6 86.1) (width 0.6) (layer "B.Cu") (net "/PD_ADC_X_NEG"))
 (segment (start 43.8 86.4) (end 42.1 84.7) (width 0.6) (layer "B.Cu") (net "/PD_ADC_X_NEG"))
 (segment (start 51.4 86.4) (end 53.1 84.7) (width 0.6) (layer "F.Cu") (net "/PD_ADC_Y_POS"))
 (segment (start 11.6 84.9) (end 13.1 86.4) (width 0.6) (layer "F.Cu") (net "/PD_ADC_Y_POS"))
 (segment (start 53.1 84.7) (end 53.1 72.7) (width 0.6) (layer "F.Cu") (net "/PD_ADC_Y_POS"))
 (segment (start 13.1 86.4) (end 51.4 86.4) (width 0.6) (layer "F.Cu") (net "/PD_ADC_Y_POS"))
 (segment (start 11.6 83.3) (end 11.6 84.9) (width 0.6) (layer "F.Cu") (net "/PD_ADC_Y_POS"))
 (segment (start 13.3 81.6) (end 11.6 83.3) (width 0.6) (layer "F.Cu") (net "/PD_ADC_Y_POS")))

